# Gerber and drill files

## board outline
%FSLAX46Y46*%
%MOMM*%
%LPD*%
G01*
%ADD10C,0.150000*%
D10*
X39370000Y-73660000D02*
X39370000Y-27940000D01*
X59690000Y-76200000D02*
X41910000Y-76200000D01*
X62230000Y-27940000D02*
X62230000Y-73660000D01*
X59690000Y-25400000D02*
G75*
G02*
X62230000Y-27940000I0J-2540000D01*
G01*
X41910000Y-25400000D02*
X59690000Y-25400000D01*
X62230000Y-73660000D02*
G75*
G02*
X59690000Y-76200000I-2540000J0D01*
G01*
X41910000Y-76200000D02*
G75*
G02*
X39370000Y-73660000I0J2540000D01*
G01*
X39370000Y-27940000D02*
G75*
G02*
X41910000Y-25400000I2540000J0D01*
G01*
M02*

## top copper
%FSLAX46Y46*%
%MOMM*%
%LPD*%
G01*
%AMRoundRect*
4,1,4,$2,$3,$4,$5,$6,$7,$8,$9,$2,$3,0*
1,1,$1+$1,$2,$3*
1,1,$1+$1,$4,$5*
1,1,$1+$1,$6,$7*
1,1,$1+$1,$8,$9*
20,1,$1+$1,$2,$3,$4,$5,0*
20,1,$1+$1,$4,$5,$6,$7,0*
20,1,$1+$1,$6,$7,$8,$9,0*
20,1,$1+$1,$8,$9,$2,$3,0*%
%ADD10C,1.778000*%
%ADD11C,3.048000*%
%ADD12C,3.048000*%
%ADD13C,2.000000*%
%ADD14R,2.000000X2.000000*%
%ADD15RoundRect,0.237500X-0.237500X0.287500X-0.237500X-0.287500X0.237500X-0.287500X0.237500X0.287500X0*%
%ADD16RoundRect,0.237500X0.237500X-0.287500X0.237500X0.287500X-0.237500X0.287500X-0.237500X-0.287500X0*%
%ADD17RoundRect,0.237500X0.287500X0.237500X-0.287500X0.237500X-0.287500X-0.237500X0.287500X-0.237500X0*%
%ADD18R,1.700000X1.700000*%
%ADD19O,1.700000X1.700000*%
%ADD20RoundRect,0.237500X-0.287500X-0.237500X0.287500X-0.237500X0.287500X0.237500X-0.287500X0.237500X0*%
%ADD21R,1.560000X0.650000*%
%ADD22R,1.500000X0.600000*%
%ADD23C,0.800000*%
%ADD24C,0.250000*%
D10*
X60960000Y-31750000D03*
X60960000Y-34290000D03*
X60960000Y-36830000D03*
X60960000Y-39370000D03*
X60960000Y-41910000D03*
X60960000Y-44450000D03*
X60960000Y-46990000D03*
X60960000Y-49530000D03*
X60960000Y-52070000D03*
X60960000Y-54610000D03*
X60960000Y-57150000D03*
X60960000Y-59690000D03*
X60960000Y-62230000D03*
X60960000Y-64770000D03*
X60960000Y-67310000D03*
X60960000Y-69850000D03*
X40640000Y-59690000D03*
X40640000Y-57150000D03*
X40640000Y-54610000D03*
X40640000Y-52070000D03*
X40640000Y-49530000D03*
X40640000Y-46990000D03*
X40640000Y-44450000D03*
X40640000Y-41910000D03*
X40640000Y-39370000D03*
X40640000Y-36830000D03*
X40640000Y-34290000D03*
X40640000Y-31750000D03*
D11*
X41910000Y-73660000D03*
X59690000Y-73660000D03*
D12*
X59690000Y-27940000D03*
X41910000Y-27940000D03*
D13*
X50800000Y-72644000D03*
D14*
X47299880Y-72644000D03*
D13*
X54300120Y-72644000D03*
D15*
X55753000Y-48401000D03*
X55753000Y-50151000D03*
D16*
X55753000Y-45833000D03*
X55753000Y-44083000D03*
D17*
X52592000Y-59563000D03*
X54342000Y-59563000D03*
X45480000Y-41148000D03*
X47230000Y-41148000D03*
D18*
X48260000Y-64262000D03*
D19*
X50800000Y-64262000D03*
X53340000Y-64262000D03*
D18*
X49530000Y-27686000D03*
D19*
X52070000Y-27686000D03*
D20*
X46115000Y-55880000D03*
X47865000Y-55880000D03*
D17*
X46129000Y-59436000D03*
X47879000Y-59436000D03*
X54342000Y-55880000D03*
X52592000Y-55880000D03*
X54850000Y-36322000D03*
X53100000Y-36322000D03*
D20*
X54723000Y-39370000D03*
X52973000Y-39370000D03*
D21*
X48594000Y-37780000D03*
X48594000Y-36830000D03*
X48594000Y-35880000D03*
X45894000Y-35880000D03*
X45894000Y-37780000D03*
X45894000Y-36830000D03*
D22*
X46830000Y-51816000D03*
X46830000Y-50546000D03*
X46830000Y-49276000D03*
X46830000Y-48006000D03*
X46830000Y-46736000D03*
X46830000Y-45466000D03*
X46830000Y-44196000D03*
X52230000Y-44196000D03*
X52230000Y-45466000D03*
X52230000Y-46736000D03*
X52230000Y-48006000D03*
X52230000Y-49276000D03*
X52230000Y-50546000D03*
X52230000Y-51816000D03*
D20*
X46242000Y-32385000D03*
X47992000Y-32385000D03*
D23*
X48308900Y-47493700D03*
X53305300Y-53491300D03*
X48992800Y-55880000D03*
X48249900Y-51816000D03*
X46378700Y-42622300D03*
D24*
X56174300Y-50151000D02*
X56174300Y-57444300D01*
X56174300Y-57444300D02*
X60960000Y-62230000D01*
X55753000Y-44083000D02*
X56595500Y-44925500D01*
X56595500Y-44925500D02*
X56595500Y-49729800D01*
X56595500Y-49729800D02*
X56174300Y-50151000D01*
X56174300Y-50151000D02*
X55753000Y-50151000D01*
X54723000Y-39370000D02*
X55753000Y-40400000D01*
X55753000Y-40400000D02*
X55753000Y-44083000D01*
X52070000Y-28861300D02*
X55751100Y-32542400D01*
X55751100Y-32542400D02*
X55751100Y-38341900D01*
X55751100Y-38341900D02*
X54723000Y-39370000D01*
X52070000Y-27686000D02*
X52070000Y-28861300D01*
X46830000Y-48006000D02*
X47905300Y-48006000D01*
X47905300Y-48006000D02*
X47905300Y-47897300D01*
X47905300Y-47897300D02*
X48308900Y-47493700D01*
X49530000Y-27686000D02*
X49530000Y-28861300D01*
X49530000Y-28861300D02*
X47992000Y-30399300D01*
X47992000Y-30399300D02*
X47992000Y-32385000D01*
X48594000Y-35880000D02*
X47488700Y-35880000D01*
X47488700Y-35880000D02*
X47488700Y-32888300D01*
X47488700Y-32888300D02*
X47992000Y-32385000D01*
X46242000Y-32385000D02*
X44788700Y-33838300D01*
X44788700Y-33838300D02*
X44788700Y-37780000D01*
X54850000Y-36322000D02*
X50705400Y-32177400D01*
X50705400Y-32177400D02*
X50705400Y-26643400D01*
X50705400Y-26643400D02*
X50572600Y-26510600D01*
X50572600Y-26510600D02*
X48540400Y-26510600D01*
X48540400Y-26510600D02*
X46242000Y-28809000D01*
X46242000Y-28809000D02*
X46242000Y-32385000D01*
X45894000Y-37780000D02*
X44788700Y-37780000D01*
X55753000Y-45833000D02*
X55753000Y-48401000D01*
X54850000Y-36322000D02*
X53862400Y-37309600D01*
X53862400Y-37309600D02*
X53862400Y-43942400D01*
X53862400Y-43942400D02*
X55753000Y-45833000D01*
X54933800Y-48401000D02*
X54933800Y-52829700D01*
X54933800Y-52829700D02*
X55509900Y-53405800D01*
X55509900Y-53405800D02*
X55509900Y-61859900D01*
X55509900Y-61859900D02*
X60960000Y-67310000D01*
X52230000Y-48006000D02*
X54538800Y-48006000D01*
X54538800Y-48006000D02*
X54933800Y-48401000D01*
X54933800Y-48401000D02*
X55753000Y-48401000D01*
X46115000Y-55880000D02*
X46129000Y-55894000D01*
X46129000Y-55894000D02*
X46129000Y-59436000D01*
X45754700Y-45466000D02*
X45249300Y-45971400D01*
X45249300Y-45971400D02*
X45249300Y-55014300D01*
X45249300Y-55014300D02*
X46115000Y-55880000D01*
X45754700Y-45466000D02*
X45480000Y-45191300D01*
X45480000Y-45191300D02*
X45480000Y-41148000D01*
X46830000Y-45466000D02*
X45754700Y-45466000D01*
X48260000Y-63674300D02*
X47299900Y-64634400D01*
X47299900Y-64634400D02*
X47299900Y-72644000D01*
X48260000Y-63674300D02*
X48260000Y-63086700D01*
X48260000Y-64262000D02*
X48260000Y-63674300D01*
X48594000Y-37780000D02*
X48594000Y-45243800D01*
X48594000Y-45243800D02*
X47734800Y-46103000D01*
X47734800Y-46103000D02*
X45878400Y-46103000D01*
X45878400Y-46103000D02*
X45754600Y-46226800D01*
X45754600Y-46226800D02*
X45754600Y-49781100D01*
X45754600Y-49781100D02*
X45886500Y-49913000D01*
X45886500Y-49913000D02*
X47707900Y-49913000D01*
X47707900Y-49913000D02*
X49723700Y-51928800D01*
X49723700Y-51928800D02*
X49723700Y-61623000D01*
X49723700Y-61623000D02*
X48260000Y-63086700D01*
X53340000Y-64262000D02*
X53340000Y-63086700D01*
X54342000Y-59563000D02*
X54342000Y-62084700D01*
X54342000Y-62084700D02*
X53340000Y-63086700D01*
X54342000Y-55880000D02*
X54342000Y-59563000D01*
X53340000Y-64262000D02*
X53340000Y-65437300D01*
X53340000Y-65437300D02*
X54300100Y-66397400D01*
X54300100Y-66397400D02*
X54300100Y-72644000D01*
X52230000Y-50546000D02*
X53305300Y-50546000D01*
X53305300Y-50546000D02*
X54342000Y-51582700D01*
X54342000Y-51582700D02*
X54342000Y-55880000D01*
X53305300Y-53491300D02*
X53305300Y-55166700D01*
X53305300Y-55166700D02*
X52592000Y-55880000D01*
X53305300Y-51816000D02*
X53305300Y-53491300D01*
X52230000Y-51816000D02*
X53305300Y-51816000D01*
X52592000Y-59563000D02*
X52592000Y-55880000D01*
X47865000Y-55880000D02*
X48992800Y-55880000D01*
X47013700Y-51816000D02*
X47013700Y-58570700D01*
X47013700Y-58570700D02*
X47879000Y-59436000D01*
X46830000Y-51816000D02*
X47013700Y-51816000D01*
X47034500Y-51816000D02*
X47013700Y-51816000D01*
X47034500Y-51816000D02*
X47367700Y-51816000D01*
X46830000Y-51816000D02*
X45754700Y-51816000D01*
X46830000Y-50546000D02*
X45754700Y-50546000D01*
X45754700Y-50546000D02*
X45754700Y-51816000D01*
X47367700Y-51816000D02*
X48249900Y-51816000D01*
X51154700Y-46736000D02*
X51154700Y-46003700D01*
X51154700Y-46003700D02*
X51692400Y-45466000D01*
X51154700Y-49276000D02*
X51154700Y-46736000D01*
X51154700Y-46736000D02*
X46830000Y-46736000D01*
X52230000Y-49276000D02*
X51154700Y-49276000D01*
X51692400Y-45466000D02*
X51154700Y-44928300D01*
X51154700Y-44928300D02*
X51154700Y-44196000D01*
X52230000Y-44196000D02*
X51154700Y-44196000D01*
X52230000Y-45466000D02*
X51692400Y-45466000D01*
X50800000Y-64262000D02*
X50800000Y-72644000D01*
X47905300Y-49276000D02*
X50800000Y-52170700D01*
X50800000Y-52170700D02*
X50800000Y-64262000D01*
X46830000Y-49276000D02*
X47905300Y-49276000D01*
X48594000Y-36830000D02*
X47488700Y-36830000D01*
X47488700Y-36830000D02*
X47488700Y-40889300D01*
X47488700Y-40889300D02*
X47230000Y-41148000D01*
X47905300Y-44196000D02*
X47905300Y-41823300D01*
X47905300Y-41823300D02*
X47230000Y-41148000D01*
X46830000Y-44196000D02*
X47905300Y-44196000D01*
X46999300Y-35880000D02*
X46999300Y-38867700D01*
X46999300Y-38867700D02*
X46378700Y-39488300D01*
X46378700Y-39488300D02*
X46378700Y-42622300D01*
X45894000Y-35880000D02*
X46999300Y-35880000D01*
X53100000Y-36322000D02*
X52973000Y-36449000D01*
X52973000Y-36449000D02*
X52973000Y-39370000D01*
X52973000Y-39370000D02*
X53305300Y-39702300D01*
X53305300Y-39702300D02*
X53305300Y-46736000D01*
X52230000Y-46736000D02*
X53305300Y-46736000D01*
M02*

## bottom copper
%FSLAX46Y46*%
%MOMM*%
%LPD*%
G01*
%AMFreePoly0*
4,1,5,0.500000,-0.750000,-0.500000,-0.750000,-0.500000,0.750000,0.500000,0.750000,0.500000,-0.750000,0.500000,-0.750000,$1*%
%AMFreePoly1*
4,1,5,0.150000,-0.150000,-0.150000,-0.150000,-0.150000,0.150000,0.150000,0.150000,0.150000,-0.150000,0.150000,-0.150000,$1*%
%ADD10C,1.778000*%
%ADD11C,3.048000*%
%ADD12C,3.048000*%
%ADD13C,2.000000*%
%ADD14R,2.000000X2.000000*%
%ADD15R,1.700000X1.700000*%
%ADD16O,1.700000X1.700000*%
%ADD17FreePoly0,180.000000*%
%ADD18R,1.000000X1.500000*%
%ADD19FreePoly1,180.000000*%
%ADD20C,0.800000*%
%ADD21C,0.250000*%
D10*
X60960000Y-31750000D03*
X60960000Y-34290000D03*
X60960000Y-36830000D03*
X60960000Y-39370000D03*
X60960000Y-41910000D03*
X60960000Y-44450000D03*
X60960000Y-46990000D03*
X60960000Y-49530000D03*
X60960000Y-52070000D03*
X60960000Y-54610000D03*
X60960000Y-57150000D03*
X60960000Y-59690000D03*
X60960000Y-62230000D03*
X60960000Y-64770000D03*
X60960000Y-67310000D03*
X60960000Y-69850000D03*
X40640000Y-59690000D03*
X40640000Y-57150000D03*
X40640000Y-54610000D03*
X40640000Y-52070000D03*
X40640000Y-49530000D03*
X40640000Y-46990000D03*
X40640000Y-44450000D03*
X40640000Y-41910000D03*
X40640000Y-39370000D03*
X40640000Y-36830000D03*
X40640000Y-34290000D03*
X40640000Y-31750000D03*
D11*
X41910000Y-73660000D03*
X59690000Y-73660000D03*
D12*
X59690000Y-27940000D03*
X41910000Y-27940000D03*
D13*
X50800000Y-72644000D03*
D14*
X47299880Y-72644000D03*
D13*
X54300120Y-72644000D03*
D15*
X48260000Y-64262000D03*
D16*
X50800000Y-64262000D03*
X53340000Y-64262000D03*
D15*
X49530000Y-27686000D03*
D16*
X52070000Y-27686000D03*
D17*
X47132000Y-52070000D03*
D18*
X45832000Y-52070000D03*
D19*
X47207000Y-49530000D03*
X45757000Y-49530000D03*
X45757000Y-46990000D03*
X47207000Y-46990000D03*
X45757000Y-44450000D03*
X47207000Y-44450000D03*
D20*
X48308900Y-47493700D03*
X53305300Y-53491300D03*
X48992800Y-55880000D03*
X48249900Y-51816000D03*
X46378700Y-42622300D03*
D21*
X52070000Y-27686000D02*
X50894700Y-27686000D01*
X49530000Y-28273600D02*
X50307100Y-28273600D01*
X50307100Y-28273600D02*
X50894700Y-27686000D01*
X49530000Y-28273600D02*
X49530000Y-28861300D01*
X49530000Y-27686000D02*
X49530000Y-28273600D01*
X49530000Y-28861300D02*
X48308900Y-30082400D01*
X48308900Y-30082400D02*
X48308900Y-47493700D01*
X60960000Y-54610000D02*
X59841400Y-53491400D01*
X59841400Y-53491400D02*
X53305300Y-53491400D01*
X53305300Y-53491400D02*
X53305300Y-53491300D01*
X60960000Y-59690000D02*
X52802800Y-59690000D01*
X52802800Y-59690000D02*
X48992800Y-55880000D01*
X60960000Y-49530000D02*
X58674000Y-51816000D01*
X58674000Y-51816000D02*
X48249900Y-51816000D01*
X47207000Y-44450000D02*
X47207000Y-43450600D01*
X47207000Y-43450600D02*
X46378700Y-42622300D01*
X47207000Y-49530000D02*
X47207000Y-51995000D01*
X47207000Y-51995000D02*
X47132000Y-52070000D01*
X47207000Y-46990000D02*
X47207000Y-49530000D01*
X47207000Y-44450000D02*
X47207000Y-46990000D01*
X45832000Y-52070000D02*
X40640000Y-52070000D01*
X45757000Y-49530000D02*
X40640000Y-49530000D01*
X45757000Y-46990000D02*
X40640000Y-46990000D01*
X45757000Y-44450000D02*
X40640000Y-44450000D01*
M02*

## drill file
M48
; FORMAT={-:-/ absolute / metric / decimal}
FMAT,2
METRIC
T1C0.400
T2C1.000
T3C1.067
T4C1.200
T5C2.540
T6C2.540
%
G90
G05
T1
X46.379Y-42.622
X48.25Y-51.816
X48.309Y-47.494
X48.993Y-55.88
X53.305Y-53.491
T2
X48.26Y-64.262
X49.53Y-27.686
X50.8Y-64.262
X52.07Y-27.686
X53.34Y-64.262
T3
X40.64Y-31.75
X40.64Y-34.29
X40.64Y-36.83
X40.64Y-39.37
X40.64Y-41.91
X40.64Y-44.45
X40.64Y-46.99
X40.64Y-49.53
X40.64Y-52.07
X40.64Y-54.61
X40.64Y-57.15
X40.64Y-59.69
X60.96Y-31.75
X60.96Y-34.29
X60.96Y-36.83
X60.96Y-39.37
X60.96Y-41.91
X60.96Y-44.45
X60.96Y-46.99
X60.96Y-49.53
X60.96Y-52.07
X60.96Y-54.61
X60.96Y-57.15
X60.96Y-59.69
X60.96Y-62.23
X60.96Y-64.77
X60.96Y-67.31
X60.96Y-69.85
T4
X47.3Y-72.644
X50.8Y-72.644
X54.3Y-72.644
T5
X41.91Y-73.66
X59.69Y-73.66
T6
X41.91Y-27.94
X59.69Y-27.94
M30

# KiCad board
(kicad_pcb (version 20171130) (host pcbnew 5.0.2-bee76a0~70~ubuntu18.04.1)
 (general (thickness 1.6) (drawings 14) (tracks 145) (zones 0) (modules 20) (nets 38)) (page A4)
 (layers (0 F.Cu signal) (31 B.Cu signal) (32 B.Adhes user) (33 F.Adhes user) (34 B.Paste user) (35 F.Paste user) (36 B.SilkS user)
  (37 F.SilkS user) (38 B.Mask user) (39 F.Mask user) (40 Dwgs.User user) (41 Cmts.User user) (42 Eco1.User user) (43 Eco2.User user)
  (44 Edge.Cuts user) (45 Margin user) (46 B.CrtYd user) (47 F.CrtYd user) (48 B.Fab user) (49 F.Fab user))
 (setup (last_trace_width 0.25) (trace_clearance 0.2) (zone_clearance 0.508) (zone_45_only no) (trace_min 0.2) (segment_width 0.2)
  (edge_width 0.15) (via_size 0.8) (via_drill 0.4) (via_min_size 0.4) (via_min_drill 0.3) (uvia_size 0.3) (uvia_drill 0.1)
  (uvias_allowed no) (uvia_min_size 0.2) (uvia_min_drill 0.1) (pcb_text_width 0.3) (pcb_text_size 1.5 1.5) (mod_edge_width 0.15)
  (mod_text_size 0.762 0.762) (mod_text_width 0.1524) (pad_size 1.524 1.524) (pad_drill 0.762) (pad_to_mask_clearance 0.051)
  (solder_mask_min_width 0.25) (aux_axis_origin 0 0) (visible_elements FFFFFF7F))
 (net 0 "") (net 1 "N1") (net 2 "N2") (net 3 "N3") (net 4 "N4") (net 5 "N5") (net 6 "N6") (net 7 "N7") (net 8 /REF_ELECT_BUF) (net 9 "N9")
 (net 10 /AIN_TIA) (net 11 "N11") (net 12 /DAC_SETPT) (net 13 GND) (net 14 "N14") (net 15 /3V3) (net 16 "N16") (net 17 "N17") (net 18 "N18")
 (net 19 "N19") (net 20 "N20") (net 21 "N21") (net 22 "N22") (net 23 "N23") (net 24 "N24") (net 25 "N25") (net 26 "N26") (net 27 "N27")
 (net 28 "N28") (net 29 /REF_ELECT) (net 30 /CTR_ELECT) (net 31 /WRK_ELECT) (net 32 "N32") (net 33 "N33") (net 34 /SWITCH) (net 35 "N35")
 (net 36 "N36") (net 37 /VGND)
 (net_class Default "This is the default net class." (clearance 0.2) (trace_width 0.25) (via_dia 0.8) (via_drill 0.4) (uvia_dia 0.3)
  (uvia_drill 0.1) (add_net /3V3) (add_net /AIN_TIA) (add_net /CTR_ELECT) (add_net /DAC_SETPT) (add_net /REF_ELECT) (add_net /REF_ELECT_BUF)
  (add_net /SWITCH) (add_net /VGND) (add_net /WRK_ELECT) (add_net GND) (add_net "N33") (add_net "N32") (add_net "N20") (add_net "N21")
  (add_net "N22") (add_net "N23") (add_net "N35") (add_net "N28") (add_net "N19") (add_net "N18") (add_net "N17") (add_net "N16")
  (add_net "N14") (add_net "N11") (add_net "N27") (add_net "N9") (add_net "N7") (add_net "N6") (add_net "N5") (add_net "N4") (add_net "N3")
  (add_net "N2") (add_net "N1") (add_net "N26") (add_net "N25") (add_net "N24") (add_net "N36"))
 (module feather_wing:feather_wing (layer F.Cu) (at 50.8 50.8)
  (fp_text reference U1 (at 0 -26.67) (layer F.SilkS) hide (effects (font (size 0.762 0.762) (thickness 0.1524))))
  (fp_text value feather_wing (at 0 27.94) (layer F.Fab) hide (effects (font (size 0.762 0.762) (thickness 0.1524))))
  (pad 28 thru_hole circle (at 10.16 -19.05) (size 1.778 1.778) (drill 1.0668) (layers *.Cu *.Mask) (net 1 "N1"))
  (pad 27 thru_hole circle (at 10.16 -16.51) (size 1.778 1.778) (drill 1.0668) (layers *.Cu *.Mask) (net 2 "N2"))
  (pad 26 thru_hole circle (at 10.16 -13.97) (size 1.778 1.778) (drill 1.0668) (layers *.Cu *.Mask) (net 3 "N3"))
  (pad 25 thru_hole circle (at 10.16 -11.43) (size 1.778 1.778) (drill 1.0668) (layers *.Cu *.Mask) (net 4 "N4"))
  (pad 24 thru_hole circle (at 10.16 -8.89) (size 1.778 1.778) (drill 1.0668) (layers *.Cu *.Mask) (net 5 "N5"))
  (pad 23 thru_hole circle (at 10.16 -6.35) (size 1.778 1.778) (drill 1.0668) (layers *.Cu *.Mask) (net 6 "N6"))
  (pad 22 thru_hole circle (at 10.16 -3.81) (size 1.778 1.778) (drill 1.0668) (layers *.Cu *.Mask) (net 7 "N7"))
  (pad 21 thru_hole circle (at 10.16 -1.27) (size 1.778 1.778) (drill 1.0668) (layers *.Cu *.Mask) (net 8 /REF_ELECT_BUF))
  (pad 20 thru_hole circle (at 10.16 1.27) (size 1.778 1.778) (drill 1.0668) (layers *.Cu *.Mask) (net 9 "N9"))
  (pad 19 thru_hole circle (at 10.16 3.81) (size 1.778 1.778) (drill 1.0668) (layers *.Cu *.Mask) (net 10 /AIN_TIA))
  (pad 18 thru_hole circle (at 10.16 6.35) (size 1.778 1.778) (drill 1.0668) (layers *.Cu *.Mask) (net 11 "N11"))
  (pad 17 thru_hole circle (at 10.16 8.89) (size 1.778 1.778) (drill 1.0668) (layers *.Cu *.Mask) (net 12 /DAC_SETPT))
  (pad 16 thru_hole circle (at 10.16 11.43) (size 1.778 1.778) (drill 1.0668) (layers *.Cu *.Mask) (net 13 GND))
  (pad 15 thru_hole circle (at 10.16 13.97) (size 1.778 1.778) (drill 1.0668) (layers *.Cu *.Mask) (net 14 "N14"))
  (pad 14 thru_hole circle (at 10.16 16.51) (size 1.778 1.778) (drill 1.0668) (layers *.Cu *.Mask) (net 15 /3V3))
  (pad 13 thru_hole circle (at 10.16 19.05) (size 1.778 1.778) (drill 1.0668) (layers *.Cu *.Mask) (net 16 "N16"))
  (pad 12 thru_hole circle (at -10.16 8.89) (size 1.778 1.778) (drill 1.0668) (layers *.Cu *.Mask) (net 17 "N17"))
  (pad 11 thru_hole circle (at -10.16 6.35) (size 1.778 1.778) (drill 1.0668) (layers *.Cu *.Mask) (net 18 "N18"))
  (pad 10 thru_hole circle (at -10.16 3.81) (size 1.778 1.778) (drill 1.0668) (layers *.Cu *.Mask) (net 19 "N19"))
  (pad 9 thru_hole circle (at -10.16 1.27) (size 1.778 1.778) (drill 1.0668) (layers *.Cu *.Mask) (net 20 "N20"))
  (pad 8 thru_hole circle (at -10.16 -1.27) (size 1.778 1.778) (drill 1.0668) (layers *.Cu *.Mask) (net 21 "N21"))
  (pad 7 thru_hole circle (at -10.16 -3.81) (size 1.778 1.778) (drill 1.0668) (layers *.Cu *.Mask) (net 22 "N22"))
  (pad 6 thru_hole circle (at -10.16 -6.35) (size 1.778 1.778) (drill 1.0668) (layers *.Cu *.Mask) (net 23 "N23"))
  (pad 5 thru_hole circle (at -10.16 -8.89) (size 1.778 1.778) (drill 1.0668) (layers *.Cu *.Mask) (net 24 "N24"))
  (pad 4 thru_hole circle (at -10.16 -11.43) (size 1.778 1.778) (drill 1.0668) (layers *.Cu *.Mask) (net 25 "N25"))
  (pad 3 thru_hole circle (at -10.16 -13.97) (size 1.778 1.778) (drill 1.0668) (layers *.Cu *.Mask) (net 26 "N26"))
  (pad 2 thru_hole circle (at -10.16 -16.51) (size 1.778 1.778) (drill 1.0668) (layers *.Cu *.Mask) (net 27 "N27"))
  (pad 1 thru_hole circle (at -10.16 -19.05) (size 1.778 1.778) (drill 1.0668) (layers *.Cu *.Mask) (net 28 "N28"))
  (pad "" thru_hole circle (at -8.89 22.86) (size 3.048 3.048) (drill 2.54) (layers *.Cu *.Mask))
  (pad "" thru_hole circle (at 8.89 22.86) (size 3.048 3.048) (drill 2.54) (layers *.Cu *.Mask))
  (pad "" np_thru_hole circle (at 8.89 -22.86) (size 3.048 3.048) (drill 2.54) (layers *.Cu *.Mask))
  (pad "" np_thru_hole circle (at -8.89 -22.86) (size 3.048 3.048) (drill 2.54) (layers *.Cu *.Mask)))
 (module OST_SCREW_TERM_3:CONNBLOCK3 (layer F.Cu) (at 50.8 72.644)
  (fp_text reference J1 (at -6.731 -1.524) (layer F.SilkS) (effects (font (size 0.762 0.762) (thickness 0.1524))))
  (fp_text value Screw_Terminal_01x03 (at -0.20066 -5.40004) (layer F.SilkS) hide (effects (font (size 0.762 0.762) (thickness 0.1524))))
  (pad 2 thru_hole circle (at 0 0) (size 2 2) (drill 1.2) (layers *.Cu *.Mask) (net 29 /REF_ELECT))
  (pad 1 thru_hole rect (at -3.50012 0) (size 2 2) (drill 1.2) (layers *.Cu *.Mask) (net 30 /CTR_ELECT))
  (pad 3 thru_hole circle (at 3.50012 0) (size 2 2) (drill 1.2) (layers *.Cu *.Mask) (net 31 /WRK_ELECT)))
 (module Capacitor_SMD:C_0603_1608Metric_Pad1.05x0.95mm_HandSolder (layer F.Cu) (at 55.753 49.276 270)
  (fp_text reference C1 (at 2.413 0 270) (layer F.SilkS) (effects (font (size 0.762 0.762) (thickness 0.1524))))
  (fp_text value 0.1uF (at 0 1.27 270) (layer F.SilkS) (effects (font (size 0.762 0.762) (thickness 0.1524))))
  (pad 1 smd roundrect (at -0.875 0 270) (size 1.05 0.95) (layers F.Cu F.Paste F.Mask) (roundrect_rratio 0.25) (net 15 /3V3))
  (pad 2 smd roundrect (at 0.875 0 270) (size 1.05 0.95) (layers F.Cu F.Paste F.Mask) (roundrect_rratio 0.25) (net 13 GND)))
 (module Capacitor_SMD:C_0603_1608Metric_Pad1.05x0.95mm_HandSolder (layer F.Cu) (at 55.753 44.958 90)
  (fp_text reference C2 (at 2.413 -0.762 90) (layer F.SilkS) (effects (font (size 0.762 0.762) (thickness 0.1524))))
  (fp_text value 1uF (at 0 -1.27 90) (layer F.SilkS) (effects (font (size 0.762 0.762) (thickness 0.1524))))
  (pad 1 smd roundrect (at -0.875 0 90) (size 1.05 0.95) (layers F.Cu F.Paste F.Mask) (roundrect_rratio 0.25) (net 15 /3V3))
  (pad 2 smd roundrect (at 0.875 0 90) (size 1.05 0.95) (layers F.Cu F.Paste F.Mask) (roundrect_rratio 0.25) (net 13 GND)))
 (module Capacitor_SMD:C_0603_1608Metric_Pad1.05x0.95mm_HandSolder (layer F.Cu) (at 53.467 59.563 180)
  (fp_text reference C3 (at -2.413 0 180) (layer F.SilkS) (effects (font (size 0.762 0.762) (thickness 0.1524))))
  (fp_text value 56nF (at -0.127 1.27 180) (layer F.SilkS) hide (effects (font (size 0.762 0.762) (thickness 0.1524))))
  (pad 2 smd roundrect (at 0.875 0 180) (size 1.05 0.95) (layers F.Cu F.Paste F.Mask) (roundrect_rratio 0.25) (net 10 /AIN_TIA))
  (pad 1 smd roundrect (at -0.875 0 180) (size 1.05 0.95) (layers F.Cu F.Paste F.Mask) (roundrect_rratio 0.25) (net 31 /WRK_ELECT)))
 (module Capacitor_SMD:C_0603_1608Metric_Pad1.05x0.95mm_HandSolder (layer F.Cu) (at 46.355 41.148 180)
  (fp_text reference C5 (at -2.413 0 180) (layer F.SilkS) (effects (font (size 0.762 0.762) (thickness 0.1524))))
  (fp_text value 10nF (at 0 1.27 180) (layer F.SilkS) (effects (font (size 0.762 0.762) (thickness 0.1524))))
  (pad 2 smd roundrect (at 0.875 0 180) (size 1.05 0.95) (layers F.Cu F.Paste F.Mask) (roundrect_rratio 0.25) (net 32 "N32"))
  (pad 1 smd roundrect (at -0.875 0 180) (size 1.05 0.95) (layers F.Cu F.Paste F.Mask) (roundrect_rratio 0.25) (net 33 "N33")))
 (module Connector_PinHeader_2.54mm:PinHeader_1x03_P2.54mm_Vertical (layer F.Cu) (at 48.26 64.262 90)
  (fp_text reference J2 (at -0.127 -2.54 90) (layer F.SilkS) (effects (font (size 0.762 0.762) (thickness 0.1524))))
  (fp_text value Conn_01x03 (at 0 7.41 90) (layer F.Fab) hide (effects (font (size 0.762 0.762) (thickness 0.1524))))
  (pad 1 thru_hole rect (at 0 0 90) (size 1.7 1.7) (drill 1) (layers *.Cu *.Mask) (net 30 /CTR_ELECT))
  (pad 2 thru_hole oval (at 0 2.54 90) (size 1.7 1.7) (drill 1) (layers *.Cu *.Mask) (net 29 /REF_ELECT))
  (pad 3 thru_hole oval (at 0 5.08 90) (size 1.7 1.7) (drill 1) (layers *.Cu *.Mask) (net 31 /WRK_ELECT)))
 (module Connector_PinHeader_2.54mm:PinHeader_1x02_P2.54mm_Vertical (layer F.Cu) (at 49.53 27.686 90)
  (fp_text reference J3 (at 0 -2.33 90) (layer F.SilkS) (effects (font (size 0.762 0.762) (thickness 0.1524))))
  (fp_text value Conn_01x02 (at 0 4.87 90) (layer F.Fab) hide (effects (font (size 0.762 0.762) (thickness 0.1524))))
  (pad 1 thru_hole rect (at 0 0 90) (size 1.7 1.7) (drill 1) (layers *.Cu *.Mask) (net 13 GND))
  (pad 2 thru_hole oval (at 0 2.54 90) (size 1.7 1.7) (drill 1) (layers *.Cu *.Mask) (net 13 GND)))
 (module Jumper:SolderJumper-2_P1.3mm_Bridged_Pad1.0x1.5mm (layer B.Cu) (at 46.482 52.07 180)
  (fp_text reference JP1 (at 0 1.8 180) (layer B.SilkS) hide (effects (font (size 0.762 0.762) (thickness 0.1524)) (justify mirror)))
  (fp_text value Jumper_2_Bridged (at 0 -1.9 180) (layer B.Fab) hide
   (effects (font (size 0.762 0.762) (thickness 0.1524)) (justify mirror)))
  (pad 1 smd custom (at -0.65 0 180) (size 1 1.5) (layers B.Cu B.Mask) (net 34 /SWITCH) (options (clearance outline) (anchor rect))
   (primitives))
  (pad 2 smd rect (at 0.65 0 180) (size 1 1.5) (layers B.Cu B.Mask) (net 20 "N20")))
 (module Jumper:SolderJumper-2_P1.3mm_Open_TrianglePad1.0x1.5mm (layer B.Cu) (at 46.482 49.53 180)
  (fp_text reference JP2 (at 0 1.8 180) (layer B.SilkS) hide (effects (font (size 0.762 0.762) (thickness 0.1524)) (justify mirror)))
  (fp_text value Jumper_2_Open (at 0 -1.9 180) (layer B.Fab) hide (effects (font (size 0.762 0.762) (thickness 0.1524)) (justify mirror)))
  (pad 1 smd custom (at -0.725 0 180) (size 0.3 0.3) (layers B.Cu B.Mask) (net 34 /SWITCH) (zone_connect 0)
   (options (clearance outline) (anchor rect)) (primitives))
  (pad 2 smd custom (at 0.725 0 180) (size 0.3 0.3) (layers B.Cu B.Mask) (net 21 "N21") (zone_connect 0)
   (options (clearance outline) (anchor rect)) (primitives)))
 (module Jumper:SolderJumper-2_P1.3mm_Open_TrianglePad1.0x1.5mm (layer B.Cu) (at 46.482 46.99 180)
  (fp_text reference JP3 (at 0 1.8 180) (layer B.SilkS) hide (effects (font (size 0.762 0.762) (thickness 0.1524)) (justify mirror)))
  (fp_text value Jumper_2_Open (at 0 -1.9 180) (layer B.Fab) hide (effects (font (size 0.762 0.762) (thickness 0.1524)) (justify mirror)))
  (pad 2 smd custom (at 0.725 0 180) (size 0.3 0.3) (layers B.Cu B.Mask) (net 22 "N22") (zone_connect 0)
   (options (clearance outline) (anchor rect)) (primitives))
  (pad 1 smd custom (at -0.725 0 180) (size 0.3 0.3) (layers B.Cu B.Mask) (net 34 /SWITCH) (zone_connect 0)
   (options (clearance outline) (anchor rect)) (primitives)))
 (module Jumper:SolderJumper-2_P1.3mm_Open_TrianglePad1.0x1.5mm (layer B.Cu) (at 46.482 44.45 180)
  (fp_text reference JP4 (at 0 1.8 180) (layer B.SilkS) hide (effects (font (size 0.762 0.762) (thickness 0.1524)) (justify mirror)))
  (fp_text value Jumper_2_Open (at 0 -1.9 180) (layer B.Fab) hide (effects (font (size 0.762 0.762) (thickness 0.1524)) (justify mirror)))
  (pad 2 smd custom (at 0.725 0 180) (size 0.3 0.3) (layers B.Cu B.Mask) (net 23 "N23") (zone_connect 0)
   (options (clearance outline) (anchor rect)) (primitives))
  (pad 1 smd custom (at -0.725 0 180) (size 0.3 0.3) (layers B.Cu B.Mask) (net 34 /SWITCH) (zone_connect 0)
   (options (clearance outline) (anchor rect)) (primitives)))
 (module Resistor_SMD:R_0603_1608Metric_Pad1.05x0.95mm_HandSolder (layer F.Cu) (at 46.99 55.88)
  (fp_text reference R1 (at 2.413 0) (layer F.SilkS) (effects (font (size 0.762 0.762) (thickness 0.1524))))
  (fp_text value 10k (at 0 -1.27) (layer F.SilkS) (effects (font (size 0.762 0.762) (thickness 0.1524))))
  (pad 1 smd roundrect (at -0.875 0) (size 1.05 0.95) (layers F.Cu F.Paste F.Mask) (roundrect_rratio 0.25) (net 32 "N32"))
  (pad 2 smd roundrect (at 0.875 0) (size 1.05 0.95) (layers F.Cu F.Paste F.Mask) (roundrect_rratio 0.25) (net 12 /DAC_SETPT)))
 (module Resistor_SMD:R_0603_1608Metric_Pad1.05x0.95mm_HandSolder (layer F.Cu) (at 47.004 59.436 180)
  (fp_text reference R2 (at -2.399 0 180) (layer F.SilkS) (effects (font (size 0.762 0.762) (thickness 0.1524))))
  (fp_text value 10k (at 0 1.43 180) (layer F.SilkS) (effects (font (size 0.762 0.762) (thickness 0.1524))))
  (pad 2 smd roundrect (at 0.875 0 180) (size 1.05 0.95) (layers F.Cu F.Paste F.Mask) (roundrect_rratio 0.25) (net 32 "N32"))
  (pad 1 smd roundrect (at -0.875 0 180) (size 1.05 0.95) (layers F.Cu F.Paste F.Mask) (roundrect_rratio 0.25) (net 8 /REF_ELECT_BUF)))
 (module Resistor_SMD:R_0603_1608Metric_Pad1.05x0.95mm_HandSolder (layer F.Cu) (at 53.467 55.88 180)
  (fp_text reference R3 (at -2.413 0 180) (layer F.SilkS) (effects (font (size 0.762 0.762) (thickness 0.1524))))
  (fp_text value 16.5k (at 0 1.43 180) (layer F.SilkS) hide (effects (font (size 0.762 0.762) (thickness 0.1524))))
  (pad 1 smd roundrect (at -0.875 0 180) (size 1.05 0.95) (layers F.Cu F.Paste F.Mask) (roundrect_rratio 0.25) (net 31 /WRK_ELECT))
  (pad 2 smd roundrect (at 0.875 0 180) (size 1.05 0.95) (layers F.Cu F.Paste F.Mask) (roundrect_rratio 0.25) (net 10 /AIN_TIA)))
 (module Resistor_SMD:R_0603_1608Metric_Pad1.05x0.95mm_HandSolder (layer F.Cu) (at 53.975 36.322 180)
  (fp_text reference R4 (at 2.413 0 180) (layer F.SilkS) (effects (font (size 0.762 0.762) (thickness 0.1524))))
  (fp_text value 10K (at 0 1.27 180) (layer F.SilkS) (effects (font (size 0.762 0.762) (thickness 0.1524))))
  (pad 1 smd roundrect (at -0.875 0 180) (size 1.05 0.95) (layers F.Cu F.Paste F.Mask) (roundrect_rratio 0.25) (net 15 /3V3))
  (pad 2 smd roundrect (at 0.875 0 180) (size 1.05 0.95) (layers F.Cu F.Paste F.Mask) (roundrect_rratio 0.25) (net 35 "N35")))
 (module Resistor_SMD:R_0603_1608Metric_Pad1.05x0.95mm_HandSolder (layer F.Cu) (at 53.848 39.37)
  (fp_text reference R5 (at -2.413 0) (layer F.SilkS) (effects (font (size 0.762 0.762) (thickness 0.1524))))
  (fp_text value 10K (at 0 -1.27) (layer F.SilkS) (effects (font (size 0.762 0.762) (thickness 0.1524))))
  (pad 2 smd roundrect (at 0.875 0) (size 1.05 0.95) (layers F.Cu F.Paste F.Mask) (roundrect_rratio 0.25) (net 13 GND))
  (pad 1 smd roundrect (at -0.875 0) (size 1.05 0.95) (layers F.Cu F.Paste F.Mask) (roundrect_rratio 0.25) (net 35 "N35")))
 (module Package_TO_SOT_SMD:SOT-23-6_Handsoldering (layer F.Cu) (at 47.244 36.83 180)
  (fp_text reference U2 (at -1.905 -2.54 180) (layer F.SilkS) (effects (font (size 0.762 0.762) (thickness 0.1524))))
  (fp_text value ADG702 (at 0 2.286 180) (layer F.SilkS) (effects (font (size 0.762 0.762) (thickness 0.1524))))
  (pad 1 smd rect (at -1.35 -0.95 180) (size 1.56 0.65) (layers F.Cu F.Paste F.Mask) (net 30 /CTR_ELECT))
  (pad 2 smd rect (at -1.35 0 180) (size 1.56 0.65) (layers F.Cu F.Paste F.Mask) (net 33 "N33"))
  (pad 3 smd rect (at -1.35 0.95 180) (size 1.56 0.65) (layers F.Cu F.Paste F.Mask) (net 13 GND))
  (pad 4 smd rect (at 1.35 0.95 180) (size 1.56 0.65) (layers F.Cu F.Paste F.Mask) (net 34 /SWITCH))
  (pad 6 smd rect (at 1.35 -0.95 180) (size 1.56 0.65) (layers F.Cu F.Paste F.Mask) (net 15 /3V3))
  (pad 5 smd rect (at 1.35 0 180) (size 1.56 0.65) (layers F.Cu F.Paste F.Mask) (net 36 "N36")))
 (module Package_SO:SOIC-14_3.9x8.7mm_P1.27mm (layer F.Cu) (at 49.53 48.006 180)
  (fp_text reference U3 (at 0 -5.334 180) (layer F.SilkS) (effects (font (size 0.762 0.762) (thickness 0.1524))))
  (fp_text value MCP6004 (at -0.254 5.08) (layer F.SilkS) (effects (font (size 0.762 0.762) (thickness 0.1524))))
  (pad 14 smd rect (at 2.7 -3.81 180) (size 1.5 0.6) (layers F.Cu F.Paste F.Mask) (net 8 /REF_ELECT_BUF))
  (pad 13 smd rect (at 2.7 -2.54 180) (size 1.5 0.6) (layers F.Cu F.Paste F.Mask) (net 8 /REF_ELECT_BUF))
  (pad 12 smd rect (at 2.7 -1.27 180) (size 1.5 0.6) (layers F.Cu F.Paste F.Mask) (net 29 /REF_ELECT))
  (pad 11 smd rect (at 2.7 0 180) (size 1.5 0.6) (layers F.Cu F.Paste F.Mask) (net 13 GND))
  (pad 10 smd rect (at 2.7 1.27 180) (size 1.5 0.6) (layers F.Cu F.Paste F.Mask) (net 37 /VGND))
  (pad 9 smd rect (at 2.7 2.54 180) (size 1.5 0.6) (layers F.Cu F.Paste F.Mask) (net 32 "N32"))
  (pad 8 smd rect (at 2.7 3.81 180) (size 1.5 0.6) (layers F.Cu F.Paste F.Mask) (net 33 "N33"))
  (pad 7 smd rect (at -2.7 3.81 180) (size 1.5 0.6) (layers F.Cu F.Paste F.Mask) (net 37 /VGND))
  (pad 6 smd rect (at -2.7 2.54 180) (size 1.5 0.6) (layers F.Cu F.Paste F.Mask) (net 37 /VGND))
  (pad 5 smd rect (at -2.7 1.27 180) (size 1.5 0.6) (layers F.Cu F.Paste F.Mask) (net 35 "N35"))
  (pad 4 smd rect (at -2.7 0 180) (size 1.5 0.6) (layers F.Cu F.Paste F.Mask) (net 15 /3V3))
  (pad 3 smd rect (at -2.7 -1.27 180) (size 1.5 0.6) (layers F.Cu F.Paste F.Mask) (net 37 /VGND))
  (pad 2 smd rect (at -2.7 -2.54 180) (size 1.5 0.6) (layers F.Cu F.Paste F.Mask) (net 31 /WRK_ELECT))
  (pad 1 smd rect (at -2.7 -3.81 180) (size 1.5 0.6) (layers F.Cu F.Paste F.Mask) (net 10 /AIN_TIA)))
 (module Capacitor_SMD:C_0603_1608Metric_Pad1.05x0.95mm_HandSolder (layer F.Cu) (at 47.117 32.385)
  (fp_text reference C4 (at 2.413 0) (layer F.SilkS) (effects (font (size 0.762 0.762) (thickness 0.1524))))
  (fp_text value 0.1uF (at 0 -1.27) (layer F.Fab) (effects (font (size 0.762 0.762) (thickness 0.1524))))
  (pad 1 smd roundrect (at -0.875 0) (size 1.05 0.95) (layers F.Cu F.Paste F.Mask) (roundrect_rratio 0.25) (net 15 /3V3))
  (pad 2 smd roundrect (at 0.875 0) (size 1.05 0.95) (layers F.Cu F.Paste F.Mask) (roundrect_rratio 0.25) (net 13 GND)))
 (gr_line (start 39.37 73.66) (end 39.37 27.94) (layer Edge.Cuts) (width 0.15))
 (gr_line (start 59.69 76.2) (end 41.91 76.2) (layer Edge.Cuts) (width 0.15))
 (gr_line (start 62.23 27.94) (end 62.23 73.66) (layer Edge.Cuts) (width 0.15))
 (gr_arc (start 59.69 27.94) (end 62.23 27.94) (angle -90) (layer Edge.Cuts) (width 0.15))
 (gr_line (start 41.91 25.4) (end 59.69 25.4) (layer Edge.Cuts) (width 0.15))
 (gr_arc (start 59.69 73.66) (end 59.69 76.2) (angle -90) (layer Edge.Cuts) (width 0.15))
 (gr_arc (start 41.91 73.66) (end 39.37 73.66) (angle -90) (layer Edge.Cuts) (width 0.15))
 (gr_arc (start 41.91 27.94) (end 41.91 25.4) (angle -90) (layer Edge.Cuts) (width 0.15))
 (segment (start 56.1743 50.151) (end 56.1743 57.4443) (width 0.25) (layer F.Cu) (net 13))
 (segment (start 56.1743 57.4443) (end 60.96 62.23) (width 0.25) (layer F.Cu) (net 13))
 (segment (start 55.753 44.083) (end 56.5955 44.9255) (width 0.25) (layer F.Cu) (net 13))
 (segment (start 56.5955 44.9255) (end 56.5955 49.7298) (width 0.25) (layer F.Cu) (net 13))
 (segment (start 56.5955 49.7298) (end 56.1743 50.151) (width 0.25) (layer F.Cu) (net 13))
 (segment (start 56.1743 50.151) (end 55.753 50.151) (width 0.25) (layer F.Cu) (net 13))
 (segment (start 54.723 39.37) (end 55.753 40.4) (width 0.25) (layer F.Cu) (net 13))
 (segment (start 55.753 40.4) (end 55.753 44.083) (width 0.25) (layer F.Cu) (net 13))
 (segment (start 52.07 28.8613) (end 55.7511 32.5424) (width 0.25) (layer F.Cu) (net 13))
 (segment (start 55.7511 32.5424) (end 55.7511 38.3419) (width 0.25) (layer F.Cu) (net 13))
 (segment (start 55.7511 38.3419) (end 54.723 39.37) (width 0.25) (layer F.Cu) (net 13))
 (segment (start 52.07 27.686) (end 52.07 28.8613) (width 0.25) (layer F.Cu) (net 13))
 (segment (start 52.07 27.686) (end 50.8947 27.686) (width 0.25) (layer B.Cu) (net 13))
 (segment (start 49.53 28.2736) (end 50.3071 28.2736) (width 0.25) (layer B.Cu) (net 13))
 (segment (start 50.3071 28.2736) (end 50.8947 27.686) (width 0.25) (layer B.Cu) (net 13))
 (segment (start 49.53 28.2736) (end 49.53 28.8613) (width 0.25) (layer B.Cu) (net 13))
 (segment (start 49.53 27.686) (end 49.53 28.2736) (width 0.25) (layer B.Cu) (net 13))
 (segment (start 46.83 48.006) (end 47.9053 48.006) (width 0.25) (layer F.Cu) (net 13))
 (segment (start 47.9053 48.006) (end 47.9053 47.8973) (width 0.25) (layer F.Cu) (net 13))
 (segment (start 47.9053 47.8973) (end 48.3089 47.4937) (width 0.25) (layer F.Cu) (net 13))
 (segment (start 49.53 28.8613) (end 48.3089 30.0824) (width 0.25) (layer B.Cu) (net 13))
 (segment (start 48.3089 30.0824) (end 48.3089 47.4937) (width 0.25) (layer B.Cu) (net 13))
 (segment (start 49.53 27.686) (end 49.53 28.8613) (width 0.25) (layer F.Cu) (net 13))
 (segment (start 49.53 28.8613) (end 47.992 30.3993) (width 0.25) (layer F.Cu) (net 13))
 (segment (start 47.992 30.3993) (end 47.992 32.385) (width 0.25) (layer F.Cu) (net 13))
 (segment (start 48.594 35.88) (end 47.4887 35.88) (width 0.25) (layer F.Cu) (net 13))
 (segment (start 47.4887 35.88) (end 47.4887 32.8883) (width 0.25) (layer F.Cu) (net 13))
 (segment (start 47.4887 32.8883) (end 47.992 32.385) (width 0.25) (layer F.Cu) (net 13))
 (via (at 48.3089 47.4937) (size 0.8) (layers F.Cu B.Cu) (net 13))
 (segment (start 46.242 32.385) (end 44.7887 33.8383) (width 0.25) (layer F.Cu) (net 15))
 (segment (start 44.7887 33.8383) (end 44.7887 37.78) (width 0.25) (layer F.Cu) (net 15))
 (segment (start 54.85 36.322) (end 50.7054 32.1774) (width 0.25) (layer F.Cu) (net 15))
 (segment (start 50.7054 32.1774) (end 50.7054 26.6434) (width 0.25) (layer F.Cu) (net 15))
 (segment (start 50.7054 26.6434) (end 50.5726 26.5106) (width 0.25) (layer F.Cu) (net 15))
 (segment (start 50.5726 26.5106) (end 48.5404 26.5106) (width 0.25) (layer F.Cu) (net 15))
 (segment (start 48.5404 26.5106) (end 46.242 28.809) (width 0.25) (layer F.Cu) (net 15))
 (segment (start 46.242 28.809) (end 46.242 32.385) (width 0.25) (layer F.Cu) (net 15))
 (segment (start 45.894 37.78) (end 44.7887 37.78) (width 0.25) (layer F.Cu) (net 15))
 (segment (start 55.753 45.833) (end 55.753 48.401) (width 0.25) (layer F.Cu) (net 15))
 (segment (start 54.85 36.322) (end 53.8624 37.3096) (width 0.25) (layer F.Cu) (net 15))
 (segment (start 53.8624 37.3096) (end 53.8624 43.9424) (width 0.25) (layer F.Cu) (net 15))
 (segment (start 53.8624 43.9424) (end 55.753 45.833) (width 0.25) (layer F.Cu) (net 15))
 (segment (start 54.9338 48.401) (end 54.9338 52.8297) (width 0.25) (layer F.Cu) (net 15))
 (segment (start 54.9338 52.8297) (end 55.5099 53.4058) (width 0.25) (layer F.Cu) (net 15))
 (segment (start 55.5099 53.4058) (end 55.5099 61.8599) (width 0.25) (layer F.Cu) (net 15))
 (segment (start 55.5099 61.8599) (end 60.96 67.31) (width 0.25) (layer F.Cu) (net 15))
 (segment (start 52.23 48.006) (end 54.5388 48.006) (width 0.25) (layer F.Cu) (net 15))
 (segment (start 54.5388 48.006) (end 54.9338 48.401) (width 0.25) (layer F.Cu) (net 15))
 (segment (start 54.9338 48.401) (end 55.753 48.401) (width 0.25) (layer F.Cu) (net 15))
 (segment (start 46.115 55.88) (end 46.129 55.894) (width 0.25) (layer F.Cu) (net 32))
 (segment (start 46.129 55.894) (end 46.129 59.436) (width 0.25) (layer F.Cu) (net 32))
 (segment (start 45.7547 45.466) (end 45.2493 45.9714) (width 0.25) (layer F.Cu) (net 32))
 (segment (start 45.2493 45.9714) (end 45.2493 55.0143) (width 0.25) (layer F.Cu) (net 32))
 (segment (start 45.2493 55.0143) (end 46.115 55.88) (width 0.25) (layer F.Cu) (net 32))
 (segment (start 45.7547 45.466) (end 45.48 45.1913) (width 0.25) (layer F.Cu) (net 32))
 (segment (start 45.48 45.1913) (end 45.48 41.148) (width 0.25) (layer F.Cu) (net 32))
 (segment (start 46.83 45.466) (end 45.7547 45.466) (width 0.25) (layer F.Cu) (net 32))
 (segment (start 48.26 63.6743) (end 47.2999 64.6344) (width 0.25) (layer F.Cu) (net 30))
 (segment (start 47.2999 64.6344) (end 47.2999 72.644) (width 0.25) (layer F.Cu) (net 30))
 (segment (start 48.26 63.6743) (end 48.26 63.0867) (width 0.25) (layer F.Cu) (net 30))
 (segment (start 48.26 64.262) (end 48.26 63.6743) (width 0.25) (layer F.Cu) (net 30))
 (segment (start 48.594 37.78) (end 48.594 45.2438) (width 0.25) (layer F.Cu) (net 30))
 (segment (start 48.594 45.2438) (end 47.7348 46.103) (width 0.25) (layer F.Cu) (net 30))
 (segment (start 47.7348 46.103) (end 45.8784 46.103) (width 0.25) (layer F.Cu) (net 30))
 (segment (start 45.8784 46.103) (end 45.7546 46.2268) (width 0.25) (layer F.Cu) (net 30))
 (segment (start 45.7546 46.2268) (end 45.7546 49.7811) (width 0.25) (layer F.Cu) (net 30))
 (segment (start 45.7546 49.7811) (end 45.8865 49.913) (width 0.25) (layer F.Cu) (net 30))
 (segment (start 45.8865 49.913) (end 47.7079 49.913) (width 0.25) (layer F.Cu) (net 30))
 (segment (start 47.7079 49.913) (end 49.7237 51.9288) (width 0.25) (layer F.Cu) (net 30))
 (segment (start 49.7237 51.9288) (end 49.7237 61.623) (width 0.25) (layer F.Cu) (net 30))
 (segment (start 49.7237 61.623) (end 48.26 63.0867) (width 0.25) (layer F.Cu) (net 30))
 (segment (start 53.34 64.262) (end 53.34 63.0867) (width 0.25) (layer F.Cu) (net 31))
 (segment (start 54.342 59.563) (end 54.342 62.0847) (width 0.25) (layer F.Cu) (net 31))
 (segment (start 54.342 62.0847) (end 53.34 63.0867) (width 0.25) (layer F.Cu) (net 31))
 (segment (start 54.342 55.88) (end 54.342 59.563) (width 0.25) (layer F.Cu) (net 31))
 (segment (start 53.34 64.262) (end 53.34 65.4373) (width 0.25) (layer F.Cu) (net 31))
 (segment (start 53.34 65.4373) (end 54.3001 66.3974) (width 0.25) (layer F.Cu) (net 31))
 (segment (start 54.3001 66.3974) (end 54.3001 72.644) (width 0.25) (layer F.Cu) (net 31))
 (segment (start 52.23 50.546) (end 53.3053 50.546) (width 0.25) (layer F.Cu) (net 31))
 (segment (start 53.3053 50.546) (end 54.342 51.5827) (width 0.25) (layer F.Cu) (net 31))
 (segment (start 54.342 51.5827) (end 54.342 55.88) (width 0.25) (layer F.Cu) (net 31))
 (segment (start 60.96 54.61) (end 59.8414 53.4914) (width 0.25) (layer B.Cu) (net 10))
 (segment (start 59.8414 53.4914) (end 53.3053 53.4914) (width 0.25) (layer B.Cu) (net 10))
 (segment (start 53.3053 53.4914) (end 53.3053 53.4913) (width 0.25) (layer B.Cu) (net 10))
 (segment (start 53.3053 53.4913) (end 53.3053 55.1667) (width 0.25) (layer F.Cu) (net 10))
 (segment (start 53.3053 55.1667) (end 52.592 55.88) (width 0.25) (layer F.Cu) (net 10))
 (segment (start 53.3053 51.816) (end 53.3053 53.4913) (width 0.25) (layer F.Cu) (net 10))
 (segment (start 52.23 51.816) (end 53.3053 51.816) (width 0.25) (layer F.Cu) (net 10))
 (segment (start 52.592 59.563) (end 52.592 55.88) (width 0.25) (layer F.Cu) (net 10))
 (via (at 53.3053 53.4913) (size 0.8) (layers F.Cu B.Cu) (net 10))
 (segment (start 47.865 55.88) (end 48.9928 55.88) (width 0.25) (layer F.Cu) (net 12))
 (segment (start 60.96 59.69) (end 52.8028 59.69) (width 0.25) (layer B.Cu) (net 12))
 (segment (start 52.8028 59.69) (end 48.9928 55.88) (width 0.25) (layer B.Cu) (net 12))
 (via (at 48.9928 55.88) (size 0.8) (layers F.Cu B.Cu) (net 12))
 (segment (start 47.0137 51.816) (end 47.0137 58.5707) (width 0.25) (layer F.Cu) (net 8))
 (segment (start 47.0137 58.5707) (end 47.879 59.436) (width 0.25) (layer F.Cu) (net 8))
 (segment (start 46.83 51.816) (end 47.0137 51.816) (width 0.25) (layer F.Cu) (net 8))
 (segment (start 47.0345 51.816) (end 47.0137 51.816) (width 0.25) (layer F.Cu) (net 8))
 (segment (start 47.0345 51.816) (end 47.3677 51.816) (width 0.25) (layer F.Cu) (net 8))
 (segment (start 46.83 51.816) (end 45.7547 51.816) (width 0.25) (layer F.Cu) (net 8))
 (segment (start 46.83 50.546) (end 45.7547 50.546) (width 0.25) (layer F.Cu) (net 8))
 (segment (start 45.7547 50.546) (end 45.7547 51.816) (width 0.25) (layer F.Cu) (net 8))
 (segment (start 47.3677 51.816) (end 48.2499 51.816) (width 0.25) (layer F.Cu) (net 8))
 (segment (start 60.96 49.53) (end 58.674 51.816) (width 0.25) (layer B.Cu) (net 8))
 (segment (start 58.674 51.816) (end 48.2499 51.816) (width 0.25) (layer B.Cu) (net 8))
 (via (at 48.2499 51.816) (size 0.8) (layers F.Cu B.Cu) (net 8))
 (segment (start 51.1547 46.736) (end 51.1547 46.0037) (width 0.25) (layer F.Cu) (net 37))
 (segment (start 51.1547 46.0037) (end 51.6924 45.466) (width 0.25) (layer F.Cu) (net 37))
 (segment (start 51.1547 49.276) (end 51.1547 46.736) (width 0.25) (layer F.Cu) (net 37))
 (segment (start 51.1547 46.736) (end 46.83 46.736) (width 0.25) (layer F.Cu) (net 37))
 (segment (start 52.23 49.276) (end 51.1547 49.276) (width 0.25) (layer F.Cu) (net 37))
 (segment (start 51.6924 45.466) (end 51.1547 44.9283) (width 0.25) (layer F.Cu) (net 37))
 (segment (start 51.1547 44.9283) (end 51.1547 44.196) (width 0.25) (layer F.Cu) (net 37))
 (segment (start 52.23 44.196) (end 51.1547 44.196) (width 0.25) (layer F.Cu) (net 37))
 (segment (start 52.23 45.466) (end 51.6924 45.466) (width 0.25) (layer F.Cu) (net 37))
 (segment (start 50.8 64.262) (end 50.8 72.644) (width 0.25) (layer F.Cu) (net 29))
 (segment (start 47.9053 49.276) (end 50.8 52.1707) (width 0.25) (layer F.Cu) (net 29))
 (segment (start 50.8 52.1707) (end 50.8 64.262) (width 0.25) (layer F.Cu) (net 29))
 (segment (start 46.83 49.276) (end 47.9053 49.276) (width 0.25) (layer F.Cu) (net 29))
 (segment (start 48.594 36.83) (end 47.4887 36.83) (width 0.25) (layer F.Cu) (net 33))
 (segment (start 47.4887 36.83) (end 47.4887 40.8893) (width 0.25) (layer F.Cu) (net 33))
 (segment (start 47.4887 40.8893) (end 47.23 41.148) (width 0.25) (layer F.Cu) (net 33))
 (segment (start 47.9053 44.196) (end 47.9053 41.8233) (width 0.25) (layer F.Cu) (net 33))
 (segment (start 47.9053 41.8233) (end 47.23 41.148) (width 0.25) (layer F.Cu) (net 33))
 (segment (start 46.83 44.196) (end 47.9053 44.196) (width 0.25) (layer F.Cu) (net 33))
 (segment (start 46.9993 35.88) (end 46.9993 38.8677) (width 0.25) (layer F.Cu) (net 34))
 (segment (start 46.9993 38.8677) (end 46.3787 39.4883) (width 0.25) (layer F.Cu) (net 34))
 (segment (start 46.3787 39.4883) (end 46.3787 42.6223) (width 0.25) (layer F.Cu) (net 34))
 (segment (start 47.207 44.45) (end 47.207 43.4506) (width 0.25) (layer B.Cu) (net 34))
 (segment (start 47.207 43.4506) (end 46.3787 42.6223) (width 0.25) (layer B.Cu) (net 34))
 (segment (start 45.894 35.88) (end 46.9993 35.88) (width 0.25) (layer F.Cu) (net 34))
 (segment (start 47.207 49.53) (end 47.207 51.995) (width 0.25) (layer B.Cu) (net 34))
 (segment (start 47.207 51.995) (end 47.132 52.07) (width 0.25) (layer B.Cu) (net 34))
 (segment (start 47.207 46.99) (end 47.207 49.53) (width 0.25) (layer B.Cu) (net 34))
 (segment (start 47.207 44.45) (end 47.207 46.99) (width 0.25) (layer B.Cu) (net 34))
 (via (at 46.3787 42.6223) (size 0.8) (layers F.Cu B.Cu) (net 34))
 (segment (start 45.832 52.07) (end 40.64 52.07) (width 0.25) (layer B.Cu) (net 20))
 (segment (start 45.757 49.53) (end 40.64 49.53) (width 0.25) (layer B.Cu) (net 21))
 (segment (start 45.757 46.99) (end 40.64 46.99) (width 0.25) (layer B.Cu) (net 22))
 (segment (start 45.757 44.45) (end 40.64 44.45) (width 0.25) (layer B.Cu) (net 23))
 (segment (start 53.1 36.322) (end 52.973 36.449) (width 0.25) (layer F.Cu) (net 35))
 (segment (start 52.973 36.449) (end 52.973 39.37) (width 0.25) (layer F.Cu) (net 35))
 (segment (start 52.973 39.37) (end 53.3053 39.7023) (width 0.25) (layer F.Cu) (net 35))
 (segment (start 53.3053 39.7023) (end 53.3053 46.736) (width 0.25) (layer F.Cu) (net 35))
 (segment (start 52.23 46.736) (end 53.3053 46.736) (width 0.25) (layer F.Cu) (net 35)))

